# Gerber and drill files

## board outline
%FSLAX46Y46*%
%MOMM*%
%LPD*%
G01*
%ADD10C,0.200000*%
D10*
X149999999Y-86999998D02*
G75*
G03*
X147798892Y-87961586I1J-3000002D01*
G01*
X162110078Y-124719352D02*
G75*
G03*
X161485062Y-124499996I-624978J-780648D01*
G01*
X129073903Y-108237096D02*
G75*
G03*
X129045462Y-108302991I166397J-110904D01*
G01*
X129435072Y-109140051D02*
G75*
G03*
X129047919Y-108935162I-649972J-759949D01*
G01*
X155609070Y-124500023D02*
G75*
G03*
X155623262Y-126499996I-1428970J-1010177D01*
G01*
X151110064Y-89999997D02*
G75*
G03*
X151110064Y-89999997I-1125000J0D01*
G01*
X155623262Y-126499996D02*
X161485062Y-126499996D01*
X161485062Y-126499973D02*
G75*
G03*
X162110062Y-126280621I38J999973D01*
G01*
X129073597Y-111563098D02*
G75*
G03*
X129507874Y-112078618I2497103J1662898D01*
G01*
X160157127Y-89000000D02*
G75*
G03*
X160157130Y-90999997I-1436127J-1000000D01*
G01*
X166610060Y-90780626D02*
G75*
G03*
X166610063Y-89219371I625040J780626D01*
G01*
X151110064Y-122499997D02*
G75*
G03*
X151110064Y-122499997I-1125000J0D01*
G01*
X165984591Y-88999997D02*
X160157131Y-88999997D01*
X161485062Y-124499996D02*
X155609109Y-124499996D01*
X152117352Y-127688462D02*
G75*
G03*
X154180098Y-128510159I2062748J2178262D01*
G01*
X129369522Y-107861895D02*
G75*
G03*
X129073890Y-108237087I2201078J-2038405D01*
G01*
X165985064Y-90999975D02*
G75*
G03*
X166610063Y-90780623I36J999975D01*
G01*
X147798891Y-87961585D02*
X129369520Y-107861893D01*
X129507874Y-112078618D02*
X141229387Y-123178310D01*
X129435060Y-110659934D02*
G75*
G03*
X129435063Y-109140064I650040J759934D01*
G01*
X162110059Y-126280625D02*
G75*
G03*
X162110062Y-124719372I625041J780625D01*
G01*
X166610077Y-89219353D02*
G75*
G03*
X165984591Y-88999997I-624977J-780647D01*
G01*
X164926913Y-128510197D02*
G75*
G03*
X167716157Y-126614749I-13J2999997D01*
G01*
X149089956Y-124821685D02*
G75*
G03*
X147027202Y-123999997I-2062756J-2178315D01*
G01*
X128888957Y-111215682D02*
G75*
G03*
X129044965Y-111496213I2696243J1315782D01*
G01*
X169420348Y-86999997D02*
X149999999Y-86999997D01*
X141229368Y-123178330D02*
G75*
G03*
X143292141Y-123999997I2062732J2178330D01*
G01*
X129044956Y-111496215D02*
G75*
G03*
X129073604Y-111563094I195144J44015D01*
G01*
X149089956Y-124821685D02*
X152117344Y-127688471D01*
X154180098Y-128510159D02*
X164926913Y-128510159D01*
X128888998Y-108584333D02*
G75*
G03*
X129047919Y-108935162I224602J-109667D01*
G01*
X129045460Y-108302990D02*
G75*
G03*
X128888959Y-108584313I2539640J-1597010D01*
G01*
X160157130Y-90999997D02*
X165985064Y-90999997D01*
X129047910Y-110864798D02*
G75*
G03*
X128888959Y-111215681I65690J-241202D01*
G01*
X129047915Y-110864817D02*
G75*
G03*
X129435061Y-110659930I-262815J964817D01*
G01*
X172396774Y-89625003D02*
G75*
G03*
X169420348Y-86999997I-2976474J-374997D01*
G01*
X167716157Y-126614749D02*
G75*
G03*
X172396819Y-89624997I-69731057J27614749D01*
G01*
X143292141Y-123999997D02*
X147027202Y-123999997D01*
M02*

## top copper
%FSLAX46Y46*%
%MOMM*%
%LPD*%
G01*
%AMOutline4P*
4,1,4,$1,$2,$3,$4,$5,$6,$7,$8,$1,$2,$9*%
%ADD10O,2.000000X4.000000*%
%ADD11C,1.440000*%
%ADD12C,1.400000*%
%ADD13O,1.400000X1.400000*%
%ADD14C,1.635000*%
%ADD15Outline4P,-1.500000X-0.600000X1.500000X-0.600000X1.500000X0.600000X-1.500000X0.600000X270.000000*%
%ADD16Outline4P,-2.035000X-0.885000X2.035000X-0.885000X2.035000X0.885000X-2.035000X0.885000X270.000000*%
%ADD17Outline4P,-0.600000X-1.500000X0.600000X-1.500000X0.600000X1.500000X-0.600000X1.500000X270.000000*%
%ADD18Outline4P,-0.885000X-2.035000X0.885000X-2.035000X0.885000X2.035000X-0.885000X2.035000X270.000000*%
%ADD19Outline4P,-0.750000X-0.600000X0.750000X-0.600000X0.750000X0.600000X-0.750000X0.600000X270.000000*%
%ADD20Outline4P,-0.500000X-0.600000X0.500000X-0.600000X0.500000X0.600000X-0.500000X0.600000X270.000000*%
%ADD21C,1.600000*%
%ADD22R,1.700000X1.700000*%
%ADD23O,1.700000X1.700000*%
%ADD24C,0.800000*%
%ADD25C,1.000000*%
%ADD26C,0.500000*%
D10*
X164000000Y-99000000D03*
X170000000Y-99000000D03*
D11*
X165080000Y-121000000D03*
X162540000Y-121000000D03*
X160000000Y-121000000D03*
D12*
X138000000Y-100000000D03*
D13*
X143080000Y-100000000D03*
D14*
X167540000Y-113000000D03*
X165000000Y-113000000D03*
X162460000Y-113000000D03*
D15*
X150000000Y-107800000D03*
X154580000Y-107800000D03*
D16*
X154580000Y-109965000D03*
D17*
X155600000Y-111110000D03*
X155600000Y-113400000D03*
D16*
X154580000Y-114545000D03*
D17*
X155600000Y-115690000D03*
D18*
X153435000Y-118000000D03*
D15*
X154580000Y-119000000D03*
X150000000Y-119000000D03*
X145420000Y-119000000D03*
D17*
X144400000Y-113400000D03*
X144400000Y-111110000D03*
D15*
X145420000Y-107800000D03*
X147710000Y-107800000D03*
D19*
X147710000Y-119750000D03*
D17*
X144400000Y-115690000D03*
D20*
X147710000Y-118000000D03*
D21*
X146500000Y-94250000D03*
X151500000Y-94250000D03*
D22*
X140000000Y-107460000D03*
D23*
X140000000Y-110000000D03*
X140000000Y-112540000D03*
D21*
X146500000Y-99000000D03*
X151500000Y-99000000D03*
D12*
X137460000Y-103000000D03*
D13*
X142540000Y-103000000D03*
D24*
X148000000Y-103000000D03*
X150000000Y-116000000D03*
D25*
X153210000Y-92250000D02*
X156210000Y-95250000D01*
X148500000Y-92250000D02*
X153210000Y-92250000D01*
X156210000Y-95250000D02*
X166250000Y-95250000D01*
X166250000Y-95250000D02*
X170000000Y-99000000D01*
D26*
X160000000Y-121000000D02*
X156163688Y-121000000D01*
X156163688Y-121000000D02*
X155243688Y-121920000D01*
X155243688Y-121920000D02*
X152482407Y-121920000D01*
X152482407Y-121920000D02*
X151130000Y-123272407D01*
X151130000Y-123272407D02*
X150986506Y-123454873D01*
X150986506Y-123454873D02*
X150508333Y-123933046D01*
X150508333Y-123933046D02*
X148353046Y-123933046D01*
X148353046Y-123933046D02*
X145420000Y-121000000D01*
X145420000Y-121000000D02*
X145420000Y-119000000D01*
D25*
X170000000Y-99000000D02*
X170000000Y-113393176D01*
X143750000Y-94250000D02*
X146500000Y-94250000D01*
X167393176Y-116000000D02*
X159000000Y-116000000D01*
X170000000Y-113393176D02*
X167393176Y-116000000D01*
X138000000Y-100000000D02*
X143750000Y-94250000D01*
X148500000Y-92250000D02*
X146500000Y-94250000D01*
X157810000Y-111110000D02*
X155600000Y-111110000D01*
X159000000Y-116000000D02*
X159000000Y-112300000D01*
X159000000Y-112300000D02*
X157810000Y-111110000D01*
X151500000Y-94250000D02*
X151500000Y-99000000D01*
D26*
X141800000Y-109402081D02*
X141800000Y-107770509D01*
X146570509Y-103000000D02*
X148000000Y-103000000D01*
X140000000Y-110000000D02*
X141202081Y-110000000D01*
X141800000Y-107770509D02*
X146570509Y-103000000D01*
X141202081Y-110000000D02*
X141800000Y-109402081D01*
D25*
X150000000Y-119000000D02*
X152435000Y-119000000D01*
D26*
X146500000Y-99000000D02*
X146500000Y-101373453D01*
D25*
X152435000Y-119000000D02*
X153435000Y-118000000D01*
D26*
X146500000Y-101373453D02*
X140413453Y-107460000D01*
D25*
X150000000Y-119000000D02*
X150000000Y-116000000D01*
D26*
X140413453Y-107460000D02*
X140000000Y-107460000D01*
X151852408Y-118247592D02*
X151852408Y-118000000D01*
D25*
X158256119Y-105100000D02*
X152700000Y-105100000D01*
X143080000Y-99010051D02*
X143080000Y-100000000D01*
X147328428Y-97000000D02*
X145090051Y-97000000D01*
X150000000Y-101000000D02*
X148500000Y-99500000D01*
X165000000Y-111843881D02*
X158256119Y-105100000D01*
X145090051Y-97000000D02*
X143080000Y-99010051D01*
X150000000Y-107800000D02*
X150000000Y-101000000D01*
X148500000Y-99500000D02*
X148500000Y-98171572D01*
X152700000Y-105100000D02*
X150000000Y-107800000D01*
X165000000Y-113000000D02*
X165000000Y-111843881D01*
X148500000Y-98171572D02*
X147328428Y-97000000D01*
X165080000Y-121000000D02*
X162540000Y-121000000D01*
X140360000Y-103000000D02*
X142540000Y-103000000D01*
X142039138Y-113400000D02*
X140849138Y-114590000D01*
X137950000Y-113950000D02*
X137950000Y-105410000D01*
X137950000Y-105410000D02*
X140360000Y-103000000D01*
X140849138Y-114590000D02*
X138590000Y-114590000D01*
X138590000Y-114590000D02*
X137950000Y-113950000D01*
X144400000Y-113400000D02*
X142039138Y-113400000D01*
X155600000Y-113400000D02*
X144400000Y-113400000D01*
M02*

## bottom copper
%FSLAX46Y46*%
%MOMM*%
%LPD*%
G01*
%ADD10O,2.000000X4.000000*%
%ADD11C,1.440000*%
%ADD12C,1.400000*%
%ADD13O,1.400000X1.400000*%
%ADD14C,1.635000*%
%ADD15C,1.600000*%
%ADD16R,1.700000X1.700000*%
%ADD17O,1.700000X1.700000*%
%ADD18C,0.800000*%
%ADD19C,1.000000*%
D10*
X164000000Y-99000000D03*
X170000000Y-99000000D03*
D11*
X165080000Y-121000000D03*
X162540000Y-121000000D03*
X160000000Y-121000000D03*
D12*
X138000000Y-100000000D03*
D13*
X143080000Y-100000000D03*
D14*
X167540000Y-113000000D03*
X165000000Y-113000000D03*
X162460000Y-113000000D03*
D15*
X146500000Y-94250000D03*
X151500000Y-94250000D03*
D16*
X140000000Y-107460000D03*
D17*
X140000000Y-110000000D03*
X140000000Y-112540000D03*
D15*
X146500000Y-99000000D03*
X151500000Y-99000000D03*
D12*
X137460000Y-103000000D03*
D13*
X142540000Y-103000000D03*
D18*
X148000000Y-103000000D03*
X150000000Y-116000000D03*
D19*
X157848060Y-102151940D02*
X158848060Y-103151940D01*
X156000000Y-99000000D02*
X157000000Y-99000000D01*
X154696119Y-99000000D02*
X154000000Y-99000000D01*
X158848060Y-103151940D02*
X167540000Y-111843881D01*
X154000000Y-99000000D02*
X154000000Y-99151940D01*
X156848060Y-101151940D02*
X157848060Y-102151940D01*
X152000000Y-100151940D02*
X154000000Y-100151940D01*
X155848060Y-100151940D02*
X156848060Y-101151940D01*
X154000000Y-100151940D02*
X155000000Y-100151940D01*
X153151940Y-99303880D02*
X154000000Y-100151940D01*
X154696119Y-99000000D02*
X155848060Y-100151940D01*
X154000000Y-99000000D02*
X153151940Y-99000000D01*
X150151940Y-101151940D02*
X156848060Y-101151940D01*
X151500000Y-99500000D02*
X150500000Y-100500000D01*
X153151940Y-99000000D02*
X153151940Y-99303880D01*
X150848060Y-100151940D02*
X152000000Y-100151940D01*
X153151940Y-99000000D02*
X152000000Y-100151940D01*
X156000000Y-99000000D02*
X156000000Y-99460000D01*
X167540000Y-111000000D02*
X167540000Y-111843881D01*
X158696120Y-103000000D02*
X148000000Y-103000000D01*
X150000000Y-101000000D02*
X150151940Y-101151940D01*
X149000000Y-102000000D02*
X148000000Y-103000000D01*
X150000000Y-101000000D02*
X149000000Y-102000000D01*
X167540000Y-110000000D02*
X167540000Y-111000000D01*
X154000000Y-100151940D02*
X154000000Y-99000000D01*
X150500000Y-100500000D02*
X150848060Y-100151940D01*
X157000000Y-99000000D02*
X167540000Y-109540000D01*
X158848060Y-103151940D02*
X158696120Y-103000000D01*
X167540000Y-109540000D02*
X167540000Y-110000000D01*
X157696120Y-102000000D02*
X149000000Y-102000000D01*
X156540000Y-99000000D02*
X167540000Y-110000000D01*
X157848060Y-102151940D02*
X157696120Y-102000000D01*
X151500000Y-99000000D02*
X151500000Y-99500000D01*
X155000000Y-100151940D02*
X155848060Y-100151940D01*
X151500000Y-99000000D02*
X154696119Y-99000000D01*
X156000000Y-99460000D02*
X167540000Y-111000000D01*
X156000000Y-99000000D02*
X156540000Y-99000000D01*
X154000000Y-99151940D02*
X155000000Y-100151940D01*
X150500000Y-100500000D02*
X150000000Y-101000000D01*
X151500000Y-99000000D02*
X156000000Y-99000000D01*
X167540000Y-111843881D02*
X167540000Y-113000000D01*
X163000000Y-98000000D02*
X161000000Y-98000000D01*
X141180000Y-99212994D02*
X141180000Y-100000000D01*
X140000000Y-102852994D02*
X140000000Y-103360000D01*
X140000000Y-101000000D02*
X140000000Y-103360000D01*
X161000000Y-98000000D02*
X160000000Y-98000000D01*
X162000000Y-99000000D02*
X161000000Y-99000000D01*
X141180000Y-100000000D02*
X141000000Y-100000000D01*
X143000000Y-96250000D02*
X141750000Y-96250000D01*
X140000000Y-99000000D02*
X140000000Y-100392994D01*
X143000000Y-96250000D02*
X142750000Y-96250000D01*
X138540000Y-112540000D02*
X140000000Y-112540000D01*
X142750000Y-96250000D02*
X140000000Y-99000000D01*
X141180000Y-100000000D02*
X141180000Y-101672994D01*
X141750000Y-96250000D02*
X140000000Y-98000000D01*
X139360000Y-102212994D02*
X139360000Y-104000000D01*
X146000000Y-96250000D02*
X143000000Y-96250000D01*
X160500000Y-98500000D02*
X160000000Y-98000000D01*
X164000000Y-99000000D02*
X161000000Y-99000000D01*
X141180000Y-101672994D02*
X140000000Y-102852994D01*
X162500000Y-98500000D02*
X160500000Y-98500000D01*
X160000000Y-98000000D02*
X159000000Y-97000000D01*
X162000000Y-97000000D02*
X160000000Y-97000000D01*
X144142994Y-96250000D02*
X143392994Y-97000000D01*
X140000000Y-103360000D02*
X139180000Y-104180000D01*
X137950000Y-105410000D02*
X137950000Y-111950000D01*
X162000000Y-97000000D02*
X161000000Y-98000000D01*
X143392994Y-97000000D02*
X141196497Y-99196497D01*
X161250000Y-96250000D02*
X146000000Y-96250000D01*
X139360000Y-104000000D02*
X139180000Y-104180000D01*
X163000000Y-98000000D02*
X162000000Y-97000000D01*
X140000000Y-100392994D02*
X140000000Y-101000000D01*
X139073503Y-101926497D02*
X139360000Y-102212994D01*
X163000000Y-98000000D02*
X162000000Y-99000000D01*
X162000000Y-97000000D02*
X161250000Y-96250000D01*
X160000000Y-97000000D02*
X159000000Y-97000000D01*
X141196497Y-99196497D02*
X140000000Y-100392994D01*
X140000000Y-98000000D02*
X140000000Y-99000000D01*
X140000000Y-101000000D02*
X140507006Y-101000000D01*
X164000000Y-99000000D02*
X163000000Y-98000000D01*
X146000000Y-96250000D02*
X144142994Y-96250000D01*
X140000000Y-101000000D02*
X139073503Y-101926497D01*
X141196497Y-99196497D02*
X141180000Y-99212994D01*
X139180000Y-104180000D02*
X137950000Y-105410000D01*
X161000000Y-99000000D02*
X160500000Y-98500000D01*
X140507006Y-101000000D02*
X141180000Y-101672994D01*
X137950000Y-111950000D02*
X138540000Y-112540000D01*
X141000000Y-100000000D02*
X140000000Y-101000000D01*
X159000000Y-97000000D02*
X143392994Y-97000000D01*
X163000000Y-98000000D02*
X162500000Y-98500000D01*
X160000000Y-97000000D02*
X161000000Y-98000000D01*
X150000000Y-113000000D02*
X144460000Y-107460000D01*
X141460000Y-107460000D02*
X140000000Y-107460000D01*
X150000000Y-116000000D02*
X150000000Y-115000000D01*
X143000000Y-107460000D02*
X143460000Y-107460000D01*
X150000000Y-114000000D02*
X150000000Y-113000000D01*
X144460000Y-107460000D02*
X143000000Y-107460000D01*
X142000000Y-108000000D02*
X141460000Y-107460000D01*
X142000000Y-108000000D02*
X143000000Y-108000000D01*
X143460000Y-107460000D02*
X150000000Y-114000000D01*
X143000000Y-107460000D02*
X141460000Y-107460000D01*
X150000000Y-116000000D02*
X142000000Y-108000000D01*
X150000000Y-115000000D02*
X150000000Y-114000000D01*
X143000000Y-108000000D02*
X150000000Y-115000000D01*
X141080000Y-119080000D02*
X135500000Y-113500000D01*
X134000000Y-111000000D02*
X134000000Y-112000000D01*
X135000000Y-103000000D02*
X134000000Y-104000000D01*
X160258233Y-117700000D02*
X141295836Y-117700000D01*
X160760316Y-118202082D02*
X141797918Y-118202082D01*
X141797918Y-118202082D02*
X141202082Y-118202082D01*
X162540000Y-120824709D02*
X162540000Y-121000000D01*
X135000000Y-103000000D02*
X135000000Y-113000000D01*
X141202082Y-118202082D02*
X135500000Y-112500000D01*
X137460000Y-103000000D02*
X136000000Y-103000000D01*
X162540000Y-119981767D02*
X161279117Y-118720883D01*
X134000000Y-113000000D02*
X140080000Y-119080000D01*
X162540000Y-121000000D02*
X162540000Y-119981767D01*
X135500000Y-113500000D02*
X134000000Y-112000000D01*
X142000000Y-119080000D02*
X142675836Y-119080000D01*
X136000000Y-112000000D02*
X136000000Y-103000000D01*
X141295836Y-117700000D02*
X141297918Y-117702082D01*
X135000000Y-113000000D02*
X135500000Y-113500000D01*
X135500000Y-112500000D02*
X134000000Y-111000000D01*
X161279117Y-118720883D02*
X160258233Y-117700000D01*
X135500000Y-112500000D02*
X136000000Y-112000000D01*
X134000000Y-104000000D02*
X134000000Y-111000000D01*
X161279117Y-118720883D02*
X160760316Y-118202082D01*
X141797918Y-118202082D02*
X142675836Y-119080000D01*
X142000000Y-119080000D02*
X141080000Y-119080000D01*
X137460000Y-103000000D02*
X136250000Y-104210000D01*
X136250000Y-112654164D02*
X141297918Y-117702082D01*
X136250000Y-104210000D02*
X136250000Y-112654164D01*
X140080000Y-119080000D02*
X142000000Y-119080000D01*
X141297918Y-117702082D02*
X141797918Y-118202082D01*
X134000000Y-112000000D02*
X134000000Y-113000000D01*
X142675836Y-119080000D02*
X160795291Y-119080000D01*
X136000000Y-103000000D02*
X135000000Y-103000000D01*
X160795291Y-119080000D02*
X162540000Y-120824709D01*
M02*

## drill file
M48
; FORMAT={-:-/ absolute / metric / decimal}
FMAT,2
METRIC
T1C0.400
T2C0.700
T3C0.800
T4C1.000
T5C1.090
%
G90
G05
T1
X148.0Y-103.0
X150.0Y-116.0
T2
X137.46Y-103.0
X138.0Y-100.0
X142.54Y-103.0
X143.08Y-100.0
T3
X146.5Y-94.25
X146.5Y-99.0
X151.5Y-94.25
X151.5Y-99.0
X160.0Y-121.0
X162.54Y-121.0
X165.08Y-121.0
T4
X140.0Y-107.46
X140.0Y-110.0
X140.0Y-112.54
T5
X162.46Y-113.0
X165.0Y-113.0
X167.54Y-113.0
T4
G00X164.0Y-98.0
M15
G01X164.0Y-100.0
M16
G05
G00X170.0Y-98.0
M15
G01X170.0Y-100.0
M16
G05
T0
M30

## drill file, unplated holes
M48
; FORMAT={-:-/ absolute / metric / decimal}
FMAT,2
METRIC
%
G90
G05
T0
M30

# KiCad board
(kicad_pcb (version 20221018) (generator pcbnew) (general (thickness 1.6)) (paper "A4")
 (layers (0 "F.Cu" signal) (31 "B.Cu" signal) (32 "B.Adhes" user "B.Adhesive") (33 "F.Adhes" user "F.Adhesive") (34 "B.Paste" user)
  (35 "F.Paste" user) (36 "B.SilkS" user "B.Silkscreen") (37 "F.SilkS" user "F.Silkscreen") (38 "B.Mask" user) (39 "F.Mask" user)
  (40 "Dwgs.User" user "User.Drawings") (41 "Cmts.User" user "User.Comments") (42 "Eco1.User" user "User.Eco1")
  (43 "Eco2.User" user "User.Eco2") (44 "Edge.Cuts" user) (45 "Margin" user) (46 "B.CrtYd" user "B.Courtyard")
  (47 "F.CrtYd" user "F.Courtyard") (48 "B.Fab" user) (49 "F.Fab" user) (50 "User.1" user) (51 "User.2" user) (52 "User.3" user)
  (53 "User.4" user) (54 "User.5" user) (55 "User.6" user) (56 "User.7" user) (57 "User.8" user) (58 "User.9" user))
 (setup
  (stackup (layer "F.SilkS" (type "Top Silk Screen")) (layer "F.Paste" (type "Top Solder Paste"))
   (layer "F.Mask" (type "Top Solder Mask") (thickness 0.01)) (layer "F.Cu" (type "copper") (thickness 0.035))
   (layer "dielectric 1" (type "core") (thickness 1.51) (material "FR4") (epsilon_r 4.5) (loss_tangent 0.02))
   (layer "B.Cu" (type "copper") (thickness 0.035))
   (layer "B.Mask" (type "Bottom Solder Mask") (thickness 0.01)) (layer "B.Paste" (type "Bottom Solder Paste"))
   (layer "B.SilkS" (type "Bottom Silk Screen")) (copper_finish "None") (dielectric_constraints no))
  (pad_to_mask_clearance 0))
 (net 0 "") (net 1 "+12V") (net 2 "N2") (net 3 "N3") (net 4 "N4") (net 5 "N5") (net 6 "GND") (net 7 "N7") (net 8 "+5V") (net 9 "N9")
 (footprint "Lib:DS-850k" (layer "F.Cu") (at 164 99 180)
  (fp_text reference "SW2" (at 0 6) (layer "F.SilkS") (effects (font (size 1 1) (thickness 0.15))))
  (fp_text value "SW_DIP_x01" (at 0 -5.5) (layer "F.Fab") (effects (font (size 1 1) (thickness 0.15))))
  (pad "1" thru_hole oval (at 0 0 270) (size 4 2) (drill oval 3 1) (layers "*.Cu" "*.Mask") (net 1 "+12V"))
  (pad "2" thru_hole oval (at -6 0 270) (size 4 2) (drill oval 3 1) (layers "*.Cu" "*.Mask") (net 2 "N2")))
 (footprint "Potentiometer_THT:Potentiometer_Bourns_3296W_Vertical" (layer "F.Cu") (at 165.08 121)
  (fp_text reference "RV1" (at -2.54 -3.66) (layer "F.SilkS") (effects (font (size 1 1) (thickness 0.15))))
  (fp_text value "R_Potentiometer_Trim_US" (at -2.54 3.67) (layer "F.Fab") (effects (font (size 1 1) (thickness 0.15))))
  (pad "1" thru_hole circle (at 0 0) (size 1.44 1.44) (drill 0.8) (layers "*.Cu" "*.Mask") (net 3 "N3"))
  (pad "2" thru_hole circle (at -2.54 0) (size 1.44 1.44) (drill 0.8) (layers "*.Cu" "*.Mask") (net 3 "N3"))
  (pad "3" thru_hole circle (at -5.08 0) (size 1.44 1.44) (drill 0.8) (layers "*.Cu" "*.Mask") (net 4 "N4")))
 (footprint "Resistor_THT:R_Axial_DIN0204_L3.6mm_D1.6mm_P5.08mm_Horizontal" (layer "F.Cu") (at 138 100)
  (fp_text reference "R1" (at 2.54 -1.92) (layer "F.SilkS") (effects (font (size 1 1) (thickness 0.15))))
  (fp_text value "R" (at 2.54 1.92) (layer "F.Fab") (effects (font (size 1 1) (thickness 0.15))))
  (pad "1" thru_hole circle (at 0 0) (size 1.4 1.4) (drill 0.7) (layers "*.Cu" "*.Mask") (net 2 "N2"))
  (pad "2" thru_hole oval (at 5.08 0) (size 1.4 1.4) (drill 0.7) (layers "*.Cu" "*.Mask") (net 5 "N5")))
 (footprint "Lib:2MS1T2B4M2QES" (layer "F.Cu") (at 167.54 113 90)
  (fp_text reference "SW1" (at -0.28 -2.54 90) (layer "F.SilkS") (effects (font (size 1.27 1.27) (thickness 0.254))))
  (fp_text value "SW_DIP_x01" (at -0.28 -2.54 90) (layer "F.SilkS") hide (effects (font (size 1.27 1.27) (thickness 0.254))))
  (pad "1" thru_hole circle (at 0 0 90) (size 1.635 1.635) (drill 1.09) (layers "*.Cu" "*.Mask") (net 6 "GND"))
  (pad "2" thru_hole circle (at 0 -2.54 90) (size 1.635 1.635) (drill 1.09) (layers "*.Cu" "*.Mask") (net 5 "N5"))
  (pad "3" thru_hole circle (at 0 -5.08 90) (size 1.635 1.635) (drill 1.09) (layers "*.Cu" "*.Mask")))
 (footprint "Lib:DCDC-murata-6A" (layer "F.Cu") (at 143.9 107.3 -90)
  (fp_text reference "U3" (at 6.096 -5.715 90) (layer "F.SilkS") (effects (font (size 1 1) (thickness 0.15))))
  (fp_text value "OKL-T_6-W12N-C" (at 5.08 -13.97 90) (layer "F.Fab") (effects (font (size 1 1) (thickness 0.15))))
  (pad "1" smd trapezoid (at 0.5 -6.1 270) (size 3 1.2) (layers "F.Cu" "F.Paste" "F.Mask") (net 5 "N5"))
  (pad "2" smd trapezoid (at 0.5 -10.68 270) (size 3 1.2) (layers "F.Cu" "F.Paste" "F.Mask") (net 2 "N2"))
  (pad "2" smd trapezoid (at 2.665 -10.68 270) (size 4.07 1.77) (layers "F.Cu" "F.Paste" "F.Mask") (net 2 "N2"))
  (pad "2" smd trapezoid (at 3.81 -11.7 270) (size 1.2 3) (layers "F.Cu" "F.Paste" "F.Mask") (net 2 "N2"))
  (pad "3" smd trapezoid (at 6.1 -11.7 270) (size 1.2 3) (layers "F.Cu" "F.Paste" "F.Mask") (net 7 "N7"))
  (pad "3" smd trapezoid (at 7.245 -10.68 270) (size 4.07 1.77) (layers "F.Cu" "F.Paste" "F.Mask") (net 7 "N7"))
  (pad "3" smd trapezoid (at 8.39 -11.7 270) (size 1.2 3) (layers "F.Cu" "F.Paste" "F.Mask") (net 7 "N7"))
  (pad "4" smd trapezoid (at 10.7 -9.535 270) (size 1.77 4.07) (layers "F.Cu" "F.Paste" "F.Mask") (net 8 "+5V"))
  (pad "4" smd trapezoid (at 11.7 -10.68 270) (size 3 1.2) (layers "F.Cu" "F.Paste" "F.Mask") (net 8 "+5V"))
  (pad "5" smd trapezoid (at 11.7 -6.1 270) (size 3 1.2) (layers "F.Cu" "F.Paste" "F.Mask") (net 8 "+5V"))
  (pad "6" smd trapezoid (at 11.7 -1.52 270) (size 3 1.2) (layers "F.Cu" "F.Paste" "F.Mask") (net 4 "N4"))
  (pad "7" smd trapezoid (at 6.1 -0.5 270) (size 1.2 3) (layers "F.Cu" "F.Paste" "F.Mask") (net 7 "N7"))
  (pad "8" smd trapezoid (at 3.81 -0.5 270) (size 1.2 3) (layers "F.Cu" "F.Paste" "F.Mask"))
  (pad "9" smd trapezoid (at 0.5 -1.52 270) (size 3 1.2) (layers "F.Cu" "F.Paste" "F.Mask"))
  (pad "10" smd trapezoid (at 0.5 -3.81 270) (size 3 1.2) (layers "F.Cu" "F.Paste" "F.Mask") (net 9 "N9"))
  (pad "11" smd trapezoid (at 12.45 -3.81 270) (size 1.5 1.2) (layers "F.Cu" "F.Paste" "F.Mask"))
  (pad "12" smd trapezoid (at 8.39 -0.5 270) (size 1.2 3) (layers "F.Cu" "F.Paste" "F.Mask"))
  (pad "13" smd trapezoid (at 10.7 -3.81 270) (size 1 1.2) (layers "F.Cu" "F.Paste" "F.Mask")))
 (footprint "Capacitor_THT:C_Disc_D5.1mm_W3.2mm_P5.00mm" (layer "F.Cu") (at 146.5 94.25)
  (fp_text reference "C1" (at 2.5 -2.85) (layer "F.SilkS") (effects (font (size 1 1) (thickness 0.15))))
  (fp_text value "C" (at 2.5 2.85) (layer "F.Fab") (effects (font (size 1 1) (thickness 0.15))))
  (pad "1" thru_hole circle (at 0 0) (size 1.6 1.6) (drill 0.8) (layers "*.Cu" "*.Mask") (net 2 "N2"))
  (pad "2" thru_hole circle (at 5 0) (size 1.6 1.6) (drill 0.8) (layers "*.Cu" "*.Mask") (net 6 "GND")))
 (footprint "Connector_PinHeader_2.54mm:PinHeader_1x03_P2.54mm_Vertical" (layer "F.Cu") (at 140 107.46)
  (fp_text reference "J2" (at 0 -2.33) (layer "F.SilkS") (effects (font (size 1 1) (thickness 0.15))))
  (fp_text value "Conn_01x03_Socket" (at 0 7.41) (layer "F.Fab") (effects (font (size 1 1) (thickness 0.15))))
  (pad "1" thru_hole rect (at 0 0) (size 1.7 1.7) (drill 1) (layers "*.Cu" "*.Mask") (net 8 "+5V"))
  (pad "2" thru_hole oval (at 0 2.54) (size 1.7 1.7) (drill 1) (layers "*.Cu" "*.Mask") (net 6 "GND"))
  (pad "3" thru_hole oval (at 0 5.08) (size 1.7 1.7) (drill 1) (layers "*.Cu" "*.Mask") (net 1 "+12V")))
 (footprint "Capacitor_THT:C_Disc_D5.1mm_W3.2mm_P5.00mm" (layer "F.Cu") (at 146.5 99)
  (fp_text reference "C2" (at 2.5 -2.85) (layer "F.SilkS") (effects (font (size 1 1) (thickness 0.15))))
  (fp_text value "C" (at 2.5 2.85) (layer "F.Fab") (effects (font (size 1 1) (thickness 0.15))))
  (pad "1" thru_hole circle (at 0 0) (size 1.6 1.6) (drill 0.8) (layers "*.Cu" "*.Mask") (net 8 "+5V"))
  (pad "2" thru_hole circle (at 5 0) (size 1.6 1.6) (drill 0.8) (layers "*.Cu" "*.Mask") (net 6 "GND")))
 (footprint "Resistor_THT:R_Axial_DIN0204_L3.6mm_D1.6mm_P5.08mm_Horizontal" (layer "F.Cu") (at 137.46 103)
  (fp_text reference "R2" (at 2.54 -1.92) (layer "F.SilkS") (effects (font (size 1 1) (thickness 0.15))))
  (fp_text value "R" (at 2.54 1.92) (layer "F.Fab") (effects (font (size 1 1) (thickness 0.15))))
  (pad "1" thru_hole circle (at 0 0) (size 1.4 1.4) (drill 0.7) (layers "*.Cu" "*.Mask") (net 3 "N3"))
  (pad "2" thru_hole oval (at 5.08 0) (size 1.4 1.4) (drill 0.7) (layers "*.Cu" "*.Mask") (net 7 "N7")))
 (gr_arc (start 147.798891 87.961585) (mid 148.799007 87.250885) (end 149.999999 86.999997) (stroke (width 0.2) (type solid))
  (layer "Edge.Cuts"))
 (gr_arc (start 161.485062 124.499996) (mid 161.816253 124.556433) (end 162.110062 124.719372) (stroke (width 0.2) (type solid))
  (layer "Edge.Cuts"))
 (gr_arc (start 129.045462 108.302991) (mid 129.056695 108.268753) (end 129.073889 108.237087) (stroke (width 0.2) (type solid))
  (layer "Edge.Cuts"))
 (gr_arc (start 129.047919 108.935162) (mid 129.252847 109.016155) (end 129.435062 109.140063) (stroke (width 0.2) (type solid))
  (layer "Edge.Cuts"))
 (gr_arc (start 155.623262 126.499996) (mid 152.430141 125.522541) (end 155.609109 124.499996) (stroke (width 0.2) (type solid))
  (layer "Edge.Cuts"))
 (gr_circle (center 149.985064 89.999997) (end 148.860064 89.999997) (stroke (width 0.2) (type solid)) (fill none) (layer "Edge.Cuts"))
 (gr_line (start 155.623262 126.499996) (end 161.485062 126.499996) (stroke (width 0.2) (type solid)) (layer "Edge.Cuts"))
 (gr_arc (start 162.110062 126.280621) (mid 161.816253 126.44356) (end 161.485062 126.499996) (stroke (width 0.2) (type solid))
  (layer "Edge.Cuts"))
 (gr_arc (start 129.507874 112.078618) (mid 129.276214 111.833091) (end 129.073603 111.563094) (stroke (width 0.2) (type solid))
  (layer "Edge.Cuts"))
 (gr_arc (start 160.15713 90.999997) (mid 156.97099 89.999995) (end 160.157131 88.999997) (stroke (width 0.2) (type solid))
  (layer "Edge.Cuts"))
 (gr_arc (start 166.610063 89.219371) (mid 168.235061 89.999997) (end 166.610063 90.780623) (stroke (width 0.2) (type solid))
  (layer "Edge.Cuts"))
 (gr_circle (center 149.985064 122.499997) (end 148.860064 122.499997) (stroke (width 0.2) (type solid)) (fill none) (layer "Edge.Cuts"))
 (gr_line (start 165.984591 88.999997) (end 160.157131 88.999997) (stroke (width 0.2) (type solid)) (layer "Edge.Cuts"))
 (gr_line (start 161.485062 124.499996) (end 155.609109 124.499996) (stroke (width 0.2) (type solid)) (layer "Edge.Cuts"))
 (gr_arc (start 154.180098 128.510159) (mid 153.069904 128.297177) (end 152.117344 127.688471) (stroke (width 0.2) (type solid))
  (layer "Edge.Cuts"))
 (gr_arc (start 129.073889 108.237087) (mid 129.214225 108.043597) (end 129.36952 107.861893) (stroke (width 0.2) (type solid))
  (layer "Edge.Cuts"))
 (gr_arc (start 166.610063 90.780623) (mid 166.316255 90.943561) (end 165.985064 90.999997) (stroke (width 0.2) (type solid))
  (layer "Edge.Cuts"))
 (gr_line (start 147.798891 87.961585) (end 129.36952 107.861893) (stroke (width 0.2) (type solid)) (layer "Edge.Cuts"))
 (gr_line (start 129.507874 112.078618) (end 141.229387 123.17831) (stroke (width 0.2) (type solid)) (layer "Edge.Cuts"))
 (gr_arc (start 129.435062 109.140063) (mid 131.085062 109.899997) (end 129.435062 110.659931) (stroke (width 0.2) (type solid))
  (layer "Edge.Cuts"))
 (gr_arc (start 162.110062 124.719372) (mid 163.735062 125.499997) (end 162.110062 126.280621) (stroke (width 0.2) (type solid))
  (layer "Edge.Cuts"))
 (gr_arc (start 165.984591 88.999997) (mid 166.316031 89.056355) (end 166.610063 89.219371) (stroke (width 0.2) (type solid))
  (layer "Edge.Cuts"))
 (gr_arc (start 167.716157 126.614749) (mid 166.613067 127.991466) (end 164.926913 128.510159) (stroke (width 0.2) (type solid))
  (layer "Edge.Cuts"))
 (gr_arc (start 147.027202 123.999997) (mid 148.137396 124.212979) (end 149.089956 124.821685) (stroke (width 0.2) (type solid))
  (layer "Edge.Cuts"))
 (gr_arc (start 129.044965 111.496213) (mid 128.963207 111.358035) (end 128.888958 111.215681) (stroke (width 0.2) (type solid))
  (layer "Edge.Cuts"))
 (gr_line (start 169.420348 86.999997) (end 149.999999 86.999997) (stroke (width 0.2) (type solid)) (layer "Edge.Cuts"))
 (gr_arc (start 143.292141 123.999997) (mid 142.181947 123.787015) (end 141.229387 123.17831) (stroke (width 0.2) (type solid))
  (layer "Edge.Cuts"))
 (gr_arc (start 129.073603 111.563094) (mid 129.056217 111.530967) (end 129.044965 111.496213) (stroke (width 0.2) (type solid))
  (layer "Edge.Cuts"))
 (gr_line (start 149.089956 124.821685) (end 152.117344 127.688471) (stroke (width 0.2) (type solid)) (layer "Edge.Cuts"))
 (gr_line (start 154.180098 128.510159) (end 164.926913 128.510159) (stroke (width 0.2) (type solid)) (layer "Edge.Cuts"))
 (gr_arc (start 129.047919 108.935162) (mid 128.885915 108.797127) (end 128.888958 108.584313) (stroke (width 0.2) (type solid))
  (layer "Edge.Cuts"))
 (gr_arc (start 128.888958 108.584313) (mid 128.963434 108.441551) (end 129.045462 108.302991) (stroke (width 0.2) (type solid))
  (layer "Edge.Cuts"))
 (gr_line (start 160.15713 90.999997) (end 165.985064 90.999997) (stroke (width 0.2) (type solid)) (layer "Edge.Cuts"))
 (gr_arc (start 128.888958 111.215681) (mid 128.885916 111.002868) (end 129.047919 110.864832) (stroke (width 0.2) (type solid))
  (layer "Edge.Cuts"))
 (gr_arc (start 129.435062 110.659931) (mid 129.252847 110.783839) (end 129.047919 110.864832) (stroke (width 0.2) (type solid))
  (layer "Edge.Cuts"))
 (gr_arc (start 169.420348 86.999997) (mid 171.404662 87.749997) (end 172.396819 89.624997) (stroke (width 0.2) (type solid))
  (layer "Edge.Cuts"))
 (gr_arc (start 172.396819 89.624997) (mid 172.391721 108.415372) (end 167.716157 126.614749) (stroke (width 0.2) (type solid))
  (layer "Edge.Cuts"))
 (gr_line (start 143.292141 123.999997) (end 147.027202 123.999997) (stroke (width 0.2) (type solid)) (layer "Edge.Cuts"))
 (segment (start 170 99) (end 170 113.393176) (width 1) (layer "F.Cu") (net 2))
 (segment (start 153.21 92.25) (end 156.21 95.25) (width 1) (layer "F.Cu") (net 2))
 (segment (start 143.75 94.25) (end 146.5 94.25) (width 1) (layer "F.Cu") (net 2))
 (segment (start 156.21 95.25) (end 166.25 95.25) (width 1) (layer "F.Cu") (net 2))
 (segment (start 167.393176 116) (end 159 116) (width 1) (layer "F.Cu") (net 2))
 (segment (start 170 113.393176) (end 167.393176 116) (width 1) (layer "F.Cu") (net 2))
 (segment (start 138 100) (end 143.75 94.25) (width 1) (layer "F.Cu") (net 2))
 (segment (start 148.5 92.25) (end 146.5 94.25) (width 1) (layer "F.Cu") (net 2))
 (segment (start 157.81 111.11) (end 155.6 111.11) (width 1) (layer "F.Cu") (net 2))
 (segment (start 159 116) (end 159 112.3) (width 1) (layer "F.Cu") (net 2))
 (segment (start 148.5 92.25) (end 153.21 92.25) (width 1) (layer "F.Cu") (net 2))
 (segment (start 166.25 95.25) (end 170 99) (width 1) (layer "F.Cu") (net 2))
 (segment (start 159 112.3) (end 157.81 111.11) (width 1) (layer "F.Cu") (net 2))
 (segment (start 151.5 94.25) (end 151.5 99) (width 1) (layer "F.Cu") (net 6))
 (segment (start 141.8 109.402081) (end 141.8 107.770509) (width 0.5) (layer "F.Cu") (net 6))
 (segment (start 146.570509 103) (end 148 103) (width 0.5) (layer "F.Cu") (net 6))
 (segment (start 140 110) (end 141.202081 110) (width 0.5) (layer "F.Cu") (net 6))
 (segment (start 141.8 107.770509) (end 146.570509 103) (width 0.5) (layer "F.Cu") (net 6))
 (segment (start 141.202081 110) (end 141.8 109.402081) (width 0.5) (layer "F.Cu") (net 6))
 (via (at 148 103) (size 0.8) (drill 0.4) (layers "F.Cu" "B.Cu") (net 6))
 (segment (start 157.84806 102.15194) (end 158.84806 103.15194) (width 1) (layer "B.Cu") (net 6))
 (segment (start 156 99) (end 157 99) (width 1) (layer "B.Cu") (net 6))
 (segment (start 154.696119 99) (end 154 99) (width 1) (layer "B.Cu") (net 6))
 (segment (start 158.84806 103.15194) (end 167.54 111.843881) (width 1) (layer "B.Cu") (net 6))
 (segment (start 154 99) (end 154 99.15194) (width 1) (layer "B.Cu") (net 6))
 (segment (start 156.84806 101.15194) (end 157.84806 102.15194) (width 1) (layer "B.Cu") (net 6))
 (segment (start 152 100.15194) (end 154 100.15194) (width 1) (layer "B.Cu") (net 6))
 (segment (start 155.84806 100.15194) (end 156.84806 101.15194) (width 1) (layer "B.Cu") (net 6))
 (segment (start 154 100.15194) (end 155 100.15194) (width 1) (layer "B.Cu") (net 6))
 (segment (start 153.15194 99.30388) (end 154 100.15194) (width 1) (layer "B.Cu") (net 6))
 (segment (start 154.696119 99) (end 155.84806 100.15194) (width 1) (layer "B.Cu") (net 6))
 (segment (start 154 99) (end 153.15194 99) (width 1) (layer "B.Cu") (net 6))
 (segment (start 150.15194 101.15194) (end 156.84806 101.15194) (width 1) (layer "B.Cu") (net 6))
 (segment (start 151.5 99.5) (end 150.5 100.5) (width 1) (layer "B.Cu") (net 6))
 (segment (start 153.15194 99) (end 153.15194 99.30388) (width 1) (layer "B.Cu") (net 6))
 (segment (start 150.84806 100.15194) (end 152 100.15194) (width 1) (layer "B.Cu") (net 6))
 (segment (start 153.15194 99) (end 152 100.15194) (width 1) (layer "B.Cu") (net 6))
 (segment (start 156 99) (end 156 99.46) (width 1) (layer "B.Cu") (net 6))
 (segment (start 167.54 111) (end 167.54 111.843881) (width 1) (layer "B.Cu") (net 6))
 (segment (start 158.69612 103) (end 148 103) (width 1) (layer "B.Cu") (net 6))
 (segment (start 150 101) (end 150.15194 101.15194) (width 1) (layer "B.Cu") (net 6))
 (segment (start 149 102) (end 148 103) (width 1) (layer "B.Cu") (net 6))
 (segment (start 150 101) (end 149 102) (width 1) (layer "B.Cu") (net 6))
 (segment (start 167.54 110) (end 167.54 111) (width 1) (layer "B.Cu") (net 6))
 (segment (start 154 100.15194) (end 154 99) (width 1) (layer "B.Cu") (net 6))
 (segment (start 150.5 100.5) (end 150.84806 100.15194) (width 1) (layer "B.Cu") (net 6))
 (segment (start 157 99) (end 167.54 109.54) (width 1) (layer "B.Cu") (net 6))
 (segment (start 158.84806 103.15194) (end 158.69612 103) (width 1) (layer "B.Cu") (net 6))
 (segment (start 167.54 109.54) (end 167.54 110) (width 1) (layer "B.Cu") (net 6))
 (segment (start 157.69612 102) (end 149 102) (width 1) (layer "B.Cu") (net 6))
 (segment (start 156.54 99) (end 167.54 110) (width 1) (layer "B.Cu") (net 6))
 (segment (start 157.84806 102.15194) (end 157.69612 102) (width 1) (layer "B.Cu") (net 6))
 (segment (start 151.5 99) (end 151.5 99.5) (width 1) (layer "B.Cu") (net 6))
 (segment (start 155 100.15194) (end 155.84806 100.15194) (width 1) (layer "B.Cu") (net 6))
 (segment (start 151.5 99) (end 154.696119 99) (width 1) (layer "B.Cu") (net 6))
 (segment (start 156 99.46) (end 167.54 111) (width 1) (layer "B.Cu") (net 6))
 (segment (start 156 99) (end 156.54 99) (width 1) (layer "B.Cu") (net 6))
 (segment (start 154 99.15194) (end 155 100.15194) (width 1) (layer "B.Cu") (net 6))
 (segment (start 150.5 100.5) (end 150 101) (width 1) (layer "B.Cu") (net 6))
 (segment (start 151.5 99) (end 156 99) (width 1) (layer "B.Cu") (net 6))
 (segment (start 167.54 111.843881) (end 167.54 113) (width 1) (layer "B.Cu") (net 6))
 (segment (start 163 98) (end 161 98) (width 1) (layer "B.Cu") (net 1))
 (segment (start 141.18 99.212994) (end 141.18 100) (width 1) (layer "B.Cu") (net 1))
 (segment (start 140 102.852994) (end 140 103.36) (width 1) (layer "B.Cu") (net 1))
 (segment (start 140 101) (end 140 103.36) (width 1) (layer "B.Cu") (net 1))
 (segment (start 161 98) (end 160 98) (width 1) (layer "B.Cu") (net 1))
 (segment (start 162 99) (end 161 99) (width 1) (layer "B.Cu") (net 1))
 (segment (start 141.18 100) (end 141 100) (width 1) (layer "B.Cu") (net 1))
 (segment (start 143 96.25) (end 141.75 96.25) (width 1) (layer "B.Cu") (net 1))
 (segment (start 140 99) (end 140 100.392994) (width 1) (layer "B.Cu") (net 1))
 (segment (start 143 96.25) (end 142.75 96.25) (width 1) (layer "B.Cu") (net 1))
 (segment (start 138.54 112.54) (end 140 112.54) (width 1) (layer "B.Cu") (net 1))
 (segment (start 142.75 96.25) (end 140 99) (width 1) (layer "B.Cu") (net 1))
 (segment (start 141.18 100) (end 141.18 101.672994) (width 1) (layer "B.Cu") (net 1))
 (segment (start 141.75 96.25) (end 140 98) (width 1) (layer "B.Cu") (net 1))
 (segment (start 139.36 102.212994) (end 139.36 104) (width 1) (layer "B.Cu") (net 1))
 (segment (start 146 96.25) (end 143 96.25) (width 1) (layer "B.Cu") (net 1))
 (segment (start 160.5 98.5) (end 160 98) (width 1) (layer "B.Cu") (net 1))
 (segment (start 164 99) (end 161 99) (width 1) (layer "B.Cu") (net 1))
 (segment (start 141.18 101.672994) (end 140 102.852994) (width 1) (layer "B.Cu") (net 1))
 (segment (start 162.5 98.5) (end 160.5 98.5) (width 1) (layer "B.Cu") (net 1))
 (segment (start 160 98) (end 159 97) (width 1) (layer "B.Cu") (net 1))
 (segment (start 162 97) (end 160 97) (width 1) (layer "B.Cu") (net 1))
 (segment (start 144.142994 96.25) (end 143.392994 97) (width 1) (layer "B.Cu") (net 1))
 (segment (start 140 103.36) (end 139.18 104.18) (width 1) (layer "B.Cu") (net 1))
 (segment (start 137.95 105.41) (end 137.95 111.95) (width 1) (layer "B.Cu") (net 1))
 (segment (start 162 97) (end 161 98) (width 1) (layer "B.Cu") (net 1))
 (segment (start 143.392994 97) (end 141.196497 99.196497) (width 1) (layer "B.Cu") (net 1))
 (segment (start 161.25 96.25) (end 146 96.25) (width 1) (layer "B.Cu") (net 1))
 (segment (start 139.36 104) (end 139.18 104.18) (width 1) (layer "B.Cu") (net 1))
 (segment (start 163 98) (end 162 97) (width 1) (layer "B.Cu") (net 1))
 (segment (start 140 100.392994) (end 140 101) (width 1) (layer "B.Cu") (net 1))
 (segment (start 139.073503 101.926497) (end 139.36 102.212994) (width 1) (layer "B.Cu") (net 1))
 (segment (start 163 98) (end 162 99) (width 1) (layer "B.Cu") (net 1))
 (segment (start 162 97) (end 161.25 96.25) (width 1) (layer "B.Cu") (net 1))
 (segment (start 160 97) (end 159 97) (width 1) (layer "B.Cu") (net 1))
 (segment (start 141.196497 99.196497) (end 140 100.392994) (width 1) (layer "B.Cu") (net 1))
 (segment (start 140 98) (end 140 99) (width 1) (layer "B.Cu") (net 1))
 (segment (start 140 101) (end 140.507006 101) (width 1) (layer "B.Cu") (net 1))
 (segment (start 164 99) (end 163 98) (width 1) (layer "B.Cu") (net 1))
 (segment (start 146 96.25) (end 144.142994 96.25) (width 1) (layer "B.Cu") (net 1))
 (segment (start 140 101) (end 139.073503 101.926497) (width 1) (layer "B.Cu") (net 1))
 (segment (start 141.196497 99.196497) (end 141.18 99.212994) (width 1) (layer "B.Cu") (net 1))
 (segment (start 139.18 104.18) (end 137.95 105.41) (width 1) (layer "B.Cu") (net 1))
 (segment (start 161 99) (end 160.5 98.5) (width 1) (layer "B.Cu") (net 1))
 (segment (start 140.507006 101) (end 141.18 101.672994) (width 1) (layer "B.Cu") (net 1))
 (segment (start 137.95 111.95) (end 138.54 112.54) (width 1) (layer "B.Cu") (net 1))
 (segment (start 141 100) (end 140 101) (width 1) (layer "B.Cu") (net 1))
 (segment (start 159 97) (end 143.392994 97) (width 1) (layer "B.Cu") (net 1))
 (segment (start 163 98) (end 162.5 98.5) (width 1) (layer "B.Cu") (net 1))
 (segment (start 160 97) (end 161 98) (width 1) (layer "B.Cu") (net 1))
 (segment (start 150 119) (end 152.435 119) (width 1) (layer "F.Cu") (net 8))
 (segment (start 146.5 99) (end 146.5 101.373453) (width 0.5) (layer "F.Cu") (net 8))
 (segment (start 152.435 119) (end 153.435 118) (width 1) (layer "F.Cu") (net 8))
 (segment (start 146.5 101.373453) (end 140.413453 107.46) (width 0.5) (layer "F.Cu") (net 8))
 (segment (start 150 119) (end 150 116) (width 1) (layer "F.Cu") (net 8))
 (segment (start 140.413453 107.46) (end 140 107.46) (width 0.5) (layer "F.Cu") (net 8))
 (segment (start 151.852408 118.247592) (end 151.852408 118) (width 0.5) (layer "F.Cu") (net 8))
 (via (at 150 116) (size 0.8) (drill 0.4) (layers "F.Cu" "B.Cu") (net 8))
 (segment (start 150 113) (end 144.46 107.46) (width 1) (layer "B.Cu") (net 8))
 (segment (start 141.46 107.46) (end 140 107.46) (width 1) (layer "B.Cu") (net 8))
 (segment (start 150 116) (end 150 115) (width 1) (layer "B.Cu") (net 8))
 (segment (start 143 107.46) (end 143.46 107.46) (width 1) (layer "B.Cu") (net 8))
 (segment (start 150 114) (end 150 113) (width 1) (layer "B.Cu") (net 8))
 (segment (start 144.46 107.46) (end 143 107.46) (width 1) (layer "B.Cu") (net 8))
 (segment (start 142 108) (end 141.46 107.46) (width 1) (layer "B.Cu") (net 8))
 (segment (start 142 108) (end 143 108) (width 1) (layer "B.Cu") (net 8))
 (segment (start 143.46 107.46) (end 150 114) (width 1) (layer "B.Cu") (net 8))
 (segment (start 143 107.46) (end 141.46 107.46) (width 1) (layer "B.Cu") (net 8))
 (segment (start 150 116) (end 142 108) (width 1) (layer "B.Cu") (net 8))
 (segment (start 150 115) (end 150 114) (width 1) (layer "B.Cu") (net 8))
 (segment (start 143 108) (end 150 115) (width 1) (layer "B.Cu") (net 8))
 (segment (start 158.256119 105.1) (end 152.7 105.1) (width 1) (layer "F.Cu") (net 5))
 (segment (start 143.08 99.010051) (end 143.08 100) (width 1) (layer "F.Cu") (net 5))
 (segment (start 147.328428 97) (end 145.090051 97) (width 1) (layer "F.Cu") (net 5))
 (segment (start 150 101) (end 148.5 99.5) (width 1) (layer "F.Cu") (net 5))
 (segment (start 165 111.843881) (end 158.256119 105.1) (width 1) (layer "F.Cu") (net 5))
 (segment (start 145.090051 97) (end 143.08 99.010051) (width 1) (layer "F.Cu") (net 5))
 (segment (start 150 107.8) (end 150 101) (width 1) (layer "F.Cu") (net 5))
 (segment (start 148.5 99.5) (end 148.5 98.171572) (width 1) (layer "F.Cu") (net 5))
 (segment (start 152.7 105.1) (end 150 107.8) (width 1) (layer "F.Cu") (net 5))
 (segment (start 165 113) (end 165 111.843881) (width 1) (layer "F.Cu") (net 5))
 (segment (start 148.5 98.171572) (end 147.328428 97) (width 1) (layer "F.Cu") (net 5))
 (segment (start 165.08 121) (end 162.54 121) (width 1) (layer "F.Cu") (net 3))
 (segment (start 141.08 119.08) (end 135.5 113.5) (width 1) (layer "B.Cu") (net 3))
 (segment (start 134 111) (end 134 112) (width 1) (layer "B.Cu") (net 3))
 (segment (start 135 103) (end 134 104) (width 1) (layer "B.Cu") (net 3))
 (segment (start 160.258233 117.7) (end 141.295836 117.7) (width 1) (layer "B.Cu") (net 3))
 (segment (start 160.760316 118.202082) (end 141.797918 118.202082) (width 1) (layer "B.Cu") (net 3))
 (segment (start 141.797918 118.202082) (end 141.202082 118.202082) (width 1) (layer "B.Cu") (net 3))
 (segment (start 162.54 120.824709) (end 162.54 121) (width 1) (layer "B.Cu") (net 3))
 (segment (start 135 103) (end 135 113) (width 1) (layer "B.Cu") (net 3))
 (segment (start 141.202082 118.202082) (end 135.5 112.5) (width 1) (layer "B.Cu") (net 3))
 (segment (start 137.46 103) (end 136 103) (width 1) (layer "B.Cu") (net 3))
 (segment (start 162.54 119.981767) (end 161.279117 118.720883) (width 1) (layer "B.Cu") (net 3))
 (segment (start 134 113) (end 140.08 119.08) (width 1) (layer "B.Cu") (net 3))
 (segment (start 162.54 121) (end 162.54 119.981767) (width 1) (layer "B.Cu") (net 3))
 (segment (start 135.5 113.5) (end 134 112) (width 1) (layer "B.Cu") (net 3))
 (segment (start 142 119.08) (end 142.675836 119.08) (width 1) (layer "B.Cu") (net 3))
 (segment (start 136 112) (end 136 103) (width 1) (layer "B.Cu") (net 3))
 (segment (start 141.295836 117.7) (end 141.297918 117.702082) (width 1) (layer "B.Cu") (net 3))
 (segment (start 135 113) (end 135.5 113.5) (width 1) (layer "B.Cu") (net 3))
 (segment (start 135.5 112.5) (end 134 111) (width 1) (layer "B.Cu") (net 3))
 (segment (start 161.279117 118.720883) (end 160.258233 117.7) (width 1) (layer "B.Cu") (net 3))
 (segment (start 135.5 112.5) (end 136 112) (width 1) (layer "B.Cu") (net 3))
 (segment (start 134 104) (end 134 111) (width 1) (layer "B.Cu") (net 3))
 (segment (start 161.279117 118.720883) (end 160.760316 118.202082) (width 1) (layer "B.Cu") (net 3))
 (segment (start 141.797918 118.202082) (end 142.675836 119.08) (width 1) (layer "B.Cu") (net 3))
 (segment (start 142 119.08) (end 141.08 119.08) (width 1) (layer "B.Cu") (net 3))
 (segment (start 137.46 103) (end 136.25 104.21) (width 1) (layer "B.Cu") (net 3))
 (segment (start 136.25 112.654164) (end 141.297918 117.702082) (width 1) (layer "B.Cu") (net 3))
 (segment (start 136.25 104.21) (end 136.25 112.654164) (width 1) (layer "B.Cu") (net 3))
 (segment (start 140.08 119.08) (end 142 119.08) (width 1) (layer "B.Cu") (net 3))
 (segment (start 141.297918 117.702082) (end 141.797918 118.202082) (width 1) (layer "B.Cu") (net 3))
 (segment (start 134 112) (end 134 113) (width 1) (layer "B.Cu") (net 3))
 (segment (start 142.675836 119.08) (end 160.795291 119.08) (width 1) (layer "B.Cu") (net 3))
 (segment (start 136 103) (end 135 103) (width 1) (layer "B.Cu") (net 3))
 (segment (start 160.795291 119.08) (end 162.54 120.824709) (width 1) (layer "B.Cu") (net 3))
 (segment (start 140.36 103) (end 142.54 103) (width 1) (layer "F.Cu") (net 7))
 (segment (start 142.039138 113.4) (end 140.849138 114.59) (width 1) (layer "F.Cu") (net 7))
 (segment (start 137.95 113.95) (end 137.95 105.41) (width 1) (layer "F.Cu") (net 7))
 (segment (start 137.95 105.41) (end 140.36 103) (width 1) (layer "F.Cu") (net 7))
 (segment (start 140.849138 114.59) (end 138.59 114.59) (width 1) (layer "F.Cu") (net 7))
 (segment (start 138.59 114.59) (end 137.95 113.95) (width 1) (layer "F.Cu") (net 7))
 (segment (start 144.4 113.4) (end 142.039138 113.4) (width 1) (layer "F.Cu") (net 7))
 (segment (start 155.6 113.4) (end 144.4 113.4) (width 1) (layer "F.Cu") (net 7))
 (segment (start 152.482407 121.92) (end 151.13 123.272407) (width 0.5) (layer "F.Cu") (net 4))
 (segment (start 151.13 123.272407) (end 150.986506 123.454873) (width 0.5) (layer "F.Cu") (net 4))
 (segment (start 145.42 121) (end 145.42 119) (width 0.5) (layer "F.Cu") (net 4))
 (segment (start 155.243688 121.92) (end 152.482407 121.92) (width 0.5) (layer "F.Cu") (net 4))
 (segment (start 156.163688 121) (end 155.243688 121.92) (width 0.5) (layer "F.Cu") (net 4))
 (segment (start 160 121) (end 156.163688 121) (width 0.5) (layer "F.Cu") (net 4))
 (segment (start 150.508333 123.933046) (end 148.353046 123.933046) (width 0.5) (layer "F.Cu") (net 4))
 (segment (start 148.353046 123.933046) (end 145.42 121) (width 0.5) (layer "F.Cu") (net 4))
 (segment (start 150.986506 123.454873) (end 150.508333 123.933046) (width 0.5) (layer "F.Cu") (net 4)))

